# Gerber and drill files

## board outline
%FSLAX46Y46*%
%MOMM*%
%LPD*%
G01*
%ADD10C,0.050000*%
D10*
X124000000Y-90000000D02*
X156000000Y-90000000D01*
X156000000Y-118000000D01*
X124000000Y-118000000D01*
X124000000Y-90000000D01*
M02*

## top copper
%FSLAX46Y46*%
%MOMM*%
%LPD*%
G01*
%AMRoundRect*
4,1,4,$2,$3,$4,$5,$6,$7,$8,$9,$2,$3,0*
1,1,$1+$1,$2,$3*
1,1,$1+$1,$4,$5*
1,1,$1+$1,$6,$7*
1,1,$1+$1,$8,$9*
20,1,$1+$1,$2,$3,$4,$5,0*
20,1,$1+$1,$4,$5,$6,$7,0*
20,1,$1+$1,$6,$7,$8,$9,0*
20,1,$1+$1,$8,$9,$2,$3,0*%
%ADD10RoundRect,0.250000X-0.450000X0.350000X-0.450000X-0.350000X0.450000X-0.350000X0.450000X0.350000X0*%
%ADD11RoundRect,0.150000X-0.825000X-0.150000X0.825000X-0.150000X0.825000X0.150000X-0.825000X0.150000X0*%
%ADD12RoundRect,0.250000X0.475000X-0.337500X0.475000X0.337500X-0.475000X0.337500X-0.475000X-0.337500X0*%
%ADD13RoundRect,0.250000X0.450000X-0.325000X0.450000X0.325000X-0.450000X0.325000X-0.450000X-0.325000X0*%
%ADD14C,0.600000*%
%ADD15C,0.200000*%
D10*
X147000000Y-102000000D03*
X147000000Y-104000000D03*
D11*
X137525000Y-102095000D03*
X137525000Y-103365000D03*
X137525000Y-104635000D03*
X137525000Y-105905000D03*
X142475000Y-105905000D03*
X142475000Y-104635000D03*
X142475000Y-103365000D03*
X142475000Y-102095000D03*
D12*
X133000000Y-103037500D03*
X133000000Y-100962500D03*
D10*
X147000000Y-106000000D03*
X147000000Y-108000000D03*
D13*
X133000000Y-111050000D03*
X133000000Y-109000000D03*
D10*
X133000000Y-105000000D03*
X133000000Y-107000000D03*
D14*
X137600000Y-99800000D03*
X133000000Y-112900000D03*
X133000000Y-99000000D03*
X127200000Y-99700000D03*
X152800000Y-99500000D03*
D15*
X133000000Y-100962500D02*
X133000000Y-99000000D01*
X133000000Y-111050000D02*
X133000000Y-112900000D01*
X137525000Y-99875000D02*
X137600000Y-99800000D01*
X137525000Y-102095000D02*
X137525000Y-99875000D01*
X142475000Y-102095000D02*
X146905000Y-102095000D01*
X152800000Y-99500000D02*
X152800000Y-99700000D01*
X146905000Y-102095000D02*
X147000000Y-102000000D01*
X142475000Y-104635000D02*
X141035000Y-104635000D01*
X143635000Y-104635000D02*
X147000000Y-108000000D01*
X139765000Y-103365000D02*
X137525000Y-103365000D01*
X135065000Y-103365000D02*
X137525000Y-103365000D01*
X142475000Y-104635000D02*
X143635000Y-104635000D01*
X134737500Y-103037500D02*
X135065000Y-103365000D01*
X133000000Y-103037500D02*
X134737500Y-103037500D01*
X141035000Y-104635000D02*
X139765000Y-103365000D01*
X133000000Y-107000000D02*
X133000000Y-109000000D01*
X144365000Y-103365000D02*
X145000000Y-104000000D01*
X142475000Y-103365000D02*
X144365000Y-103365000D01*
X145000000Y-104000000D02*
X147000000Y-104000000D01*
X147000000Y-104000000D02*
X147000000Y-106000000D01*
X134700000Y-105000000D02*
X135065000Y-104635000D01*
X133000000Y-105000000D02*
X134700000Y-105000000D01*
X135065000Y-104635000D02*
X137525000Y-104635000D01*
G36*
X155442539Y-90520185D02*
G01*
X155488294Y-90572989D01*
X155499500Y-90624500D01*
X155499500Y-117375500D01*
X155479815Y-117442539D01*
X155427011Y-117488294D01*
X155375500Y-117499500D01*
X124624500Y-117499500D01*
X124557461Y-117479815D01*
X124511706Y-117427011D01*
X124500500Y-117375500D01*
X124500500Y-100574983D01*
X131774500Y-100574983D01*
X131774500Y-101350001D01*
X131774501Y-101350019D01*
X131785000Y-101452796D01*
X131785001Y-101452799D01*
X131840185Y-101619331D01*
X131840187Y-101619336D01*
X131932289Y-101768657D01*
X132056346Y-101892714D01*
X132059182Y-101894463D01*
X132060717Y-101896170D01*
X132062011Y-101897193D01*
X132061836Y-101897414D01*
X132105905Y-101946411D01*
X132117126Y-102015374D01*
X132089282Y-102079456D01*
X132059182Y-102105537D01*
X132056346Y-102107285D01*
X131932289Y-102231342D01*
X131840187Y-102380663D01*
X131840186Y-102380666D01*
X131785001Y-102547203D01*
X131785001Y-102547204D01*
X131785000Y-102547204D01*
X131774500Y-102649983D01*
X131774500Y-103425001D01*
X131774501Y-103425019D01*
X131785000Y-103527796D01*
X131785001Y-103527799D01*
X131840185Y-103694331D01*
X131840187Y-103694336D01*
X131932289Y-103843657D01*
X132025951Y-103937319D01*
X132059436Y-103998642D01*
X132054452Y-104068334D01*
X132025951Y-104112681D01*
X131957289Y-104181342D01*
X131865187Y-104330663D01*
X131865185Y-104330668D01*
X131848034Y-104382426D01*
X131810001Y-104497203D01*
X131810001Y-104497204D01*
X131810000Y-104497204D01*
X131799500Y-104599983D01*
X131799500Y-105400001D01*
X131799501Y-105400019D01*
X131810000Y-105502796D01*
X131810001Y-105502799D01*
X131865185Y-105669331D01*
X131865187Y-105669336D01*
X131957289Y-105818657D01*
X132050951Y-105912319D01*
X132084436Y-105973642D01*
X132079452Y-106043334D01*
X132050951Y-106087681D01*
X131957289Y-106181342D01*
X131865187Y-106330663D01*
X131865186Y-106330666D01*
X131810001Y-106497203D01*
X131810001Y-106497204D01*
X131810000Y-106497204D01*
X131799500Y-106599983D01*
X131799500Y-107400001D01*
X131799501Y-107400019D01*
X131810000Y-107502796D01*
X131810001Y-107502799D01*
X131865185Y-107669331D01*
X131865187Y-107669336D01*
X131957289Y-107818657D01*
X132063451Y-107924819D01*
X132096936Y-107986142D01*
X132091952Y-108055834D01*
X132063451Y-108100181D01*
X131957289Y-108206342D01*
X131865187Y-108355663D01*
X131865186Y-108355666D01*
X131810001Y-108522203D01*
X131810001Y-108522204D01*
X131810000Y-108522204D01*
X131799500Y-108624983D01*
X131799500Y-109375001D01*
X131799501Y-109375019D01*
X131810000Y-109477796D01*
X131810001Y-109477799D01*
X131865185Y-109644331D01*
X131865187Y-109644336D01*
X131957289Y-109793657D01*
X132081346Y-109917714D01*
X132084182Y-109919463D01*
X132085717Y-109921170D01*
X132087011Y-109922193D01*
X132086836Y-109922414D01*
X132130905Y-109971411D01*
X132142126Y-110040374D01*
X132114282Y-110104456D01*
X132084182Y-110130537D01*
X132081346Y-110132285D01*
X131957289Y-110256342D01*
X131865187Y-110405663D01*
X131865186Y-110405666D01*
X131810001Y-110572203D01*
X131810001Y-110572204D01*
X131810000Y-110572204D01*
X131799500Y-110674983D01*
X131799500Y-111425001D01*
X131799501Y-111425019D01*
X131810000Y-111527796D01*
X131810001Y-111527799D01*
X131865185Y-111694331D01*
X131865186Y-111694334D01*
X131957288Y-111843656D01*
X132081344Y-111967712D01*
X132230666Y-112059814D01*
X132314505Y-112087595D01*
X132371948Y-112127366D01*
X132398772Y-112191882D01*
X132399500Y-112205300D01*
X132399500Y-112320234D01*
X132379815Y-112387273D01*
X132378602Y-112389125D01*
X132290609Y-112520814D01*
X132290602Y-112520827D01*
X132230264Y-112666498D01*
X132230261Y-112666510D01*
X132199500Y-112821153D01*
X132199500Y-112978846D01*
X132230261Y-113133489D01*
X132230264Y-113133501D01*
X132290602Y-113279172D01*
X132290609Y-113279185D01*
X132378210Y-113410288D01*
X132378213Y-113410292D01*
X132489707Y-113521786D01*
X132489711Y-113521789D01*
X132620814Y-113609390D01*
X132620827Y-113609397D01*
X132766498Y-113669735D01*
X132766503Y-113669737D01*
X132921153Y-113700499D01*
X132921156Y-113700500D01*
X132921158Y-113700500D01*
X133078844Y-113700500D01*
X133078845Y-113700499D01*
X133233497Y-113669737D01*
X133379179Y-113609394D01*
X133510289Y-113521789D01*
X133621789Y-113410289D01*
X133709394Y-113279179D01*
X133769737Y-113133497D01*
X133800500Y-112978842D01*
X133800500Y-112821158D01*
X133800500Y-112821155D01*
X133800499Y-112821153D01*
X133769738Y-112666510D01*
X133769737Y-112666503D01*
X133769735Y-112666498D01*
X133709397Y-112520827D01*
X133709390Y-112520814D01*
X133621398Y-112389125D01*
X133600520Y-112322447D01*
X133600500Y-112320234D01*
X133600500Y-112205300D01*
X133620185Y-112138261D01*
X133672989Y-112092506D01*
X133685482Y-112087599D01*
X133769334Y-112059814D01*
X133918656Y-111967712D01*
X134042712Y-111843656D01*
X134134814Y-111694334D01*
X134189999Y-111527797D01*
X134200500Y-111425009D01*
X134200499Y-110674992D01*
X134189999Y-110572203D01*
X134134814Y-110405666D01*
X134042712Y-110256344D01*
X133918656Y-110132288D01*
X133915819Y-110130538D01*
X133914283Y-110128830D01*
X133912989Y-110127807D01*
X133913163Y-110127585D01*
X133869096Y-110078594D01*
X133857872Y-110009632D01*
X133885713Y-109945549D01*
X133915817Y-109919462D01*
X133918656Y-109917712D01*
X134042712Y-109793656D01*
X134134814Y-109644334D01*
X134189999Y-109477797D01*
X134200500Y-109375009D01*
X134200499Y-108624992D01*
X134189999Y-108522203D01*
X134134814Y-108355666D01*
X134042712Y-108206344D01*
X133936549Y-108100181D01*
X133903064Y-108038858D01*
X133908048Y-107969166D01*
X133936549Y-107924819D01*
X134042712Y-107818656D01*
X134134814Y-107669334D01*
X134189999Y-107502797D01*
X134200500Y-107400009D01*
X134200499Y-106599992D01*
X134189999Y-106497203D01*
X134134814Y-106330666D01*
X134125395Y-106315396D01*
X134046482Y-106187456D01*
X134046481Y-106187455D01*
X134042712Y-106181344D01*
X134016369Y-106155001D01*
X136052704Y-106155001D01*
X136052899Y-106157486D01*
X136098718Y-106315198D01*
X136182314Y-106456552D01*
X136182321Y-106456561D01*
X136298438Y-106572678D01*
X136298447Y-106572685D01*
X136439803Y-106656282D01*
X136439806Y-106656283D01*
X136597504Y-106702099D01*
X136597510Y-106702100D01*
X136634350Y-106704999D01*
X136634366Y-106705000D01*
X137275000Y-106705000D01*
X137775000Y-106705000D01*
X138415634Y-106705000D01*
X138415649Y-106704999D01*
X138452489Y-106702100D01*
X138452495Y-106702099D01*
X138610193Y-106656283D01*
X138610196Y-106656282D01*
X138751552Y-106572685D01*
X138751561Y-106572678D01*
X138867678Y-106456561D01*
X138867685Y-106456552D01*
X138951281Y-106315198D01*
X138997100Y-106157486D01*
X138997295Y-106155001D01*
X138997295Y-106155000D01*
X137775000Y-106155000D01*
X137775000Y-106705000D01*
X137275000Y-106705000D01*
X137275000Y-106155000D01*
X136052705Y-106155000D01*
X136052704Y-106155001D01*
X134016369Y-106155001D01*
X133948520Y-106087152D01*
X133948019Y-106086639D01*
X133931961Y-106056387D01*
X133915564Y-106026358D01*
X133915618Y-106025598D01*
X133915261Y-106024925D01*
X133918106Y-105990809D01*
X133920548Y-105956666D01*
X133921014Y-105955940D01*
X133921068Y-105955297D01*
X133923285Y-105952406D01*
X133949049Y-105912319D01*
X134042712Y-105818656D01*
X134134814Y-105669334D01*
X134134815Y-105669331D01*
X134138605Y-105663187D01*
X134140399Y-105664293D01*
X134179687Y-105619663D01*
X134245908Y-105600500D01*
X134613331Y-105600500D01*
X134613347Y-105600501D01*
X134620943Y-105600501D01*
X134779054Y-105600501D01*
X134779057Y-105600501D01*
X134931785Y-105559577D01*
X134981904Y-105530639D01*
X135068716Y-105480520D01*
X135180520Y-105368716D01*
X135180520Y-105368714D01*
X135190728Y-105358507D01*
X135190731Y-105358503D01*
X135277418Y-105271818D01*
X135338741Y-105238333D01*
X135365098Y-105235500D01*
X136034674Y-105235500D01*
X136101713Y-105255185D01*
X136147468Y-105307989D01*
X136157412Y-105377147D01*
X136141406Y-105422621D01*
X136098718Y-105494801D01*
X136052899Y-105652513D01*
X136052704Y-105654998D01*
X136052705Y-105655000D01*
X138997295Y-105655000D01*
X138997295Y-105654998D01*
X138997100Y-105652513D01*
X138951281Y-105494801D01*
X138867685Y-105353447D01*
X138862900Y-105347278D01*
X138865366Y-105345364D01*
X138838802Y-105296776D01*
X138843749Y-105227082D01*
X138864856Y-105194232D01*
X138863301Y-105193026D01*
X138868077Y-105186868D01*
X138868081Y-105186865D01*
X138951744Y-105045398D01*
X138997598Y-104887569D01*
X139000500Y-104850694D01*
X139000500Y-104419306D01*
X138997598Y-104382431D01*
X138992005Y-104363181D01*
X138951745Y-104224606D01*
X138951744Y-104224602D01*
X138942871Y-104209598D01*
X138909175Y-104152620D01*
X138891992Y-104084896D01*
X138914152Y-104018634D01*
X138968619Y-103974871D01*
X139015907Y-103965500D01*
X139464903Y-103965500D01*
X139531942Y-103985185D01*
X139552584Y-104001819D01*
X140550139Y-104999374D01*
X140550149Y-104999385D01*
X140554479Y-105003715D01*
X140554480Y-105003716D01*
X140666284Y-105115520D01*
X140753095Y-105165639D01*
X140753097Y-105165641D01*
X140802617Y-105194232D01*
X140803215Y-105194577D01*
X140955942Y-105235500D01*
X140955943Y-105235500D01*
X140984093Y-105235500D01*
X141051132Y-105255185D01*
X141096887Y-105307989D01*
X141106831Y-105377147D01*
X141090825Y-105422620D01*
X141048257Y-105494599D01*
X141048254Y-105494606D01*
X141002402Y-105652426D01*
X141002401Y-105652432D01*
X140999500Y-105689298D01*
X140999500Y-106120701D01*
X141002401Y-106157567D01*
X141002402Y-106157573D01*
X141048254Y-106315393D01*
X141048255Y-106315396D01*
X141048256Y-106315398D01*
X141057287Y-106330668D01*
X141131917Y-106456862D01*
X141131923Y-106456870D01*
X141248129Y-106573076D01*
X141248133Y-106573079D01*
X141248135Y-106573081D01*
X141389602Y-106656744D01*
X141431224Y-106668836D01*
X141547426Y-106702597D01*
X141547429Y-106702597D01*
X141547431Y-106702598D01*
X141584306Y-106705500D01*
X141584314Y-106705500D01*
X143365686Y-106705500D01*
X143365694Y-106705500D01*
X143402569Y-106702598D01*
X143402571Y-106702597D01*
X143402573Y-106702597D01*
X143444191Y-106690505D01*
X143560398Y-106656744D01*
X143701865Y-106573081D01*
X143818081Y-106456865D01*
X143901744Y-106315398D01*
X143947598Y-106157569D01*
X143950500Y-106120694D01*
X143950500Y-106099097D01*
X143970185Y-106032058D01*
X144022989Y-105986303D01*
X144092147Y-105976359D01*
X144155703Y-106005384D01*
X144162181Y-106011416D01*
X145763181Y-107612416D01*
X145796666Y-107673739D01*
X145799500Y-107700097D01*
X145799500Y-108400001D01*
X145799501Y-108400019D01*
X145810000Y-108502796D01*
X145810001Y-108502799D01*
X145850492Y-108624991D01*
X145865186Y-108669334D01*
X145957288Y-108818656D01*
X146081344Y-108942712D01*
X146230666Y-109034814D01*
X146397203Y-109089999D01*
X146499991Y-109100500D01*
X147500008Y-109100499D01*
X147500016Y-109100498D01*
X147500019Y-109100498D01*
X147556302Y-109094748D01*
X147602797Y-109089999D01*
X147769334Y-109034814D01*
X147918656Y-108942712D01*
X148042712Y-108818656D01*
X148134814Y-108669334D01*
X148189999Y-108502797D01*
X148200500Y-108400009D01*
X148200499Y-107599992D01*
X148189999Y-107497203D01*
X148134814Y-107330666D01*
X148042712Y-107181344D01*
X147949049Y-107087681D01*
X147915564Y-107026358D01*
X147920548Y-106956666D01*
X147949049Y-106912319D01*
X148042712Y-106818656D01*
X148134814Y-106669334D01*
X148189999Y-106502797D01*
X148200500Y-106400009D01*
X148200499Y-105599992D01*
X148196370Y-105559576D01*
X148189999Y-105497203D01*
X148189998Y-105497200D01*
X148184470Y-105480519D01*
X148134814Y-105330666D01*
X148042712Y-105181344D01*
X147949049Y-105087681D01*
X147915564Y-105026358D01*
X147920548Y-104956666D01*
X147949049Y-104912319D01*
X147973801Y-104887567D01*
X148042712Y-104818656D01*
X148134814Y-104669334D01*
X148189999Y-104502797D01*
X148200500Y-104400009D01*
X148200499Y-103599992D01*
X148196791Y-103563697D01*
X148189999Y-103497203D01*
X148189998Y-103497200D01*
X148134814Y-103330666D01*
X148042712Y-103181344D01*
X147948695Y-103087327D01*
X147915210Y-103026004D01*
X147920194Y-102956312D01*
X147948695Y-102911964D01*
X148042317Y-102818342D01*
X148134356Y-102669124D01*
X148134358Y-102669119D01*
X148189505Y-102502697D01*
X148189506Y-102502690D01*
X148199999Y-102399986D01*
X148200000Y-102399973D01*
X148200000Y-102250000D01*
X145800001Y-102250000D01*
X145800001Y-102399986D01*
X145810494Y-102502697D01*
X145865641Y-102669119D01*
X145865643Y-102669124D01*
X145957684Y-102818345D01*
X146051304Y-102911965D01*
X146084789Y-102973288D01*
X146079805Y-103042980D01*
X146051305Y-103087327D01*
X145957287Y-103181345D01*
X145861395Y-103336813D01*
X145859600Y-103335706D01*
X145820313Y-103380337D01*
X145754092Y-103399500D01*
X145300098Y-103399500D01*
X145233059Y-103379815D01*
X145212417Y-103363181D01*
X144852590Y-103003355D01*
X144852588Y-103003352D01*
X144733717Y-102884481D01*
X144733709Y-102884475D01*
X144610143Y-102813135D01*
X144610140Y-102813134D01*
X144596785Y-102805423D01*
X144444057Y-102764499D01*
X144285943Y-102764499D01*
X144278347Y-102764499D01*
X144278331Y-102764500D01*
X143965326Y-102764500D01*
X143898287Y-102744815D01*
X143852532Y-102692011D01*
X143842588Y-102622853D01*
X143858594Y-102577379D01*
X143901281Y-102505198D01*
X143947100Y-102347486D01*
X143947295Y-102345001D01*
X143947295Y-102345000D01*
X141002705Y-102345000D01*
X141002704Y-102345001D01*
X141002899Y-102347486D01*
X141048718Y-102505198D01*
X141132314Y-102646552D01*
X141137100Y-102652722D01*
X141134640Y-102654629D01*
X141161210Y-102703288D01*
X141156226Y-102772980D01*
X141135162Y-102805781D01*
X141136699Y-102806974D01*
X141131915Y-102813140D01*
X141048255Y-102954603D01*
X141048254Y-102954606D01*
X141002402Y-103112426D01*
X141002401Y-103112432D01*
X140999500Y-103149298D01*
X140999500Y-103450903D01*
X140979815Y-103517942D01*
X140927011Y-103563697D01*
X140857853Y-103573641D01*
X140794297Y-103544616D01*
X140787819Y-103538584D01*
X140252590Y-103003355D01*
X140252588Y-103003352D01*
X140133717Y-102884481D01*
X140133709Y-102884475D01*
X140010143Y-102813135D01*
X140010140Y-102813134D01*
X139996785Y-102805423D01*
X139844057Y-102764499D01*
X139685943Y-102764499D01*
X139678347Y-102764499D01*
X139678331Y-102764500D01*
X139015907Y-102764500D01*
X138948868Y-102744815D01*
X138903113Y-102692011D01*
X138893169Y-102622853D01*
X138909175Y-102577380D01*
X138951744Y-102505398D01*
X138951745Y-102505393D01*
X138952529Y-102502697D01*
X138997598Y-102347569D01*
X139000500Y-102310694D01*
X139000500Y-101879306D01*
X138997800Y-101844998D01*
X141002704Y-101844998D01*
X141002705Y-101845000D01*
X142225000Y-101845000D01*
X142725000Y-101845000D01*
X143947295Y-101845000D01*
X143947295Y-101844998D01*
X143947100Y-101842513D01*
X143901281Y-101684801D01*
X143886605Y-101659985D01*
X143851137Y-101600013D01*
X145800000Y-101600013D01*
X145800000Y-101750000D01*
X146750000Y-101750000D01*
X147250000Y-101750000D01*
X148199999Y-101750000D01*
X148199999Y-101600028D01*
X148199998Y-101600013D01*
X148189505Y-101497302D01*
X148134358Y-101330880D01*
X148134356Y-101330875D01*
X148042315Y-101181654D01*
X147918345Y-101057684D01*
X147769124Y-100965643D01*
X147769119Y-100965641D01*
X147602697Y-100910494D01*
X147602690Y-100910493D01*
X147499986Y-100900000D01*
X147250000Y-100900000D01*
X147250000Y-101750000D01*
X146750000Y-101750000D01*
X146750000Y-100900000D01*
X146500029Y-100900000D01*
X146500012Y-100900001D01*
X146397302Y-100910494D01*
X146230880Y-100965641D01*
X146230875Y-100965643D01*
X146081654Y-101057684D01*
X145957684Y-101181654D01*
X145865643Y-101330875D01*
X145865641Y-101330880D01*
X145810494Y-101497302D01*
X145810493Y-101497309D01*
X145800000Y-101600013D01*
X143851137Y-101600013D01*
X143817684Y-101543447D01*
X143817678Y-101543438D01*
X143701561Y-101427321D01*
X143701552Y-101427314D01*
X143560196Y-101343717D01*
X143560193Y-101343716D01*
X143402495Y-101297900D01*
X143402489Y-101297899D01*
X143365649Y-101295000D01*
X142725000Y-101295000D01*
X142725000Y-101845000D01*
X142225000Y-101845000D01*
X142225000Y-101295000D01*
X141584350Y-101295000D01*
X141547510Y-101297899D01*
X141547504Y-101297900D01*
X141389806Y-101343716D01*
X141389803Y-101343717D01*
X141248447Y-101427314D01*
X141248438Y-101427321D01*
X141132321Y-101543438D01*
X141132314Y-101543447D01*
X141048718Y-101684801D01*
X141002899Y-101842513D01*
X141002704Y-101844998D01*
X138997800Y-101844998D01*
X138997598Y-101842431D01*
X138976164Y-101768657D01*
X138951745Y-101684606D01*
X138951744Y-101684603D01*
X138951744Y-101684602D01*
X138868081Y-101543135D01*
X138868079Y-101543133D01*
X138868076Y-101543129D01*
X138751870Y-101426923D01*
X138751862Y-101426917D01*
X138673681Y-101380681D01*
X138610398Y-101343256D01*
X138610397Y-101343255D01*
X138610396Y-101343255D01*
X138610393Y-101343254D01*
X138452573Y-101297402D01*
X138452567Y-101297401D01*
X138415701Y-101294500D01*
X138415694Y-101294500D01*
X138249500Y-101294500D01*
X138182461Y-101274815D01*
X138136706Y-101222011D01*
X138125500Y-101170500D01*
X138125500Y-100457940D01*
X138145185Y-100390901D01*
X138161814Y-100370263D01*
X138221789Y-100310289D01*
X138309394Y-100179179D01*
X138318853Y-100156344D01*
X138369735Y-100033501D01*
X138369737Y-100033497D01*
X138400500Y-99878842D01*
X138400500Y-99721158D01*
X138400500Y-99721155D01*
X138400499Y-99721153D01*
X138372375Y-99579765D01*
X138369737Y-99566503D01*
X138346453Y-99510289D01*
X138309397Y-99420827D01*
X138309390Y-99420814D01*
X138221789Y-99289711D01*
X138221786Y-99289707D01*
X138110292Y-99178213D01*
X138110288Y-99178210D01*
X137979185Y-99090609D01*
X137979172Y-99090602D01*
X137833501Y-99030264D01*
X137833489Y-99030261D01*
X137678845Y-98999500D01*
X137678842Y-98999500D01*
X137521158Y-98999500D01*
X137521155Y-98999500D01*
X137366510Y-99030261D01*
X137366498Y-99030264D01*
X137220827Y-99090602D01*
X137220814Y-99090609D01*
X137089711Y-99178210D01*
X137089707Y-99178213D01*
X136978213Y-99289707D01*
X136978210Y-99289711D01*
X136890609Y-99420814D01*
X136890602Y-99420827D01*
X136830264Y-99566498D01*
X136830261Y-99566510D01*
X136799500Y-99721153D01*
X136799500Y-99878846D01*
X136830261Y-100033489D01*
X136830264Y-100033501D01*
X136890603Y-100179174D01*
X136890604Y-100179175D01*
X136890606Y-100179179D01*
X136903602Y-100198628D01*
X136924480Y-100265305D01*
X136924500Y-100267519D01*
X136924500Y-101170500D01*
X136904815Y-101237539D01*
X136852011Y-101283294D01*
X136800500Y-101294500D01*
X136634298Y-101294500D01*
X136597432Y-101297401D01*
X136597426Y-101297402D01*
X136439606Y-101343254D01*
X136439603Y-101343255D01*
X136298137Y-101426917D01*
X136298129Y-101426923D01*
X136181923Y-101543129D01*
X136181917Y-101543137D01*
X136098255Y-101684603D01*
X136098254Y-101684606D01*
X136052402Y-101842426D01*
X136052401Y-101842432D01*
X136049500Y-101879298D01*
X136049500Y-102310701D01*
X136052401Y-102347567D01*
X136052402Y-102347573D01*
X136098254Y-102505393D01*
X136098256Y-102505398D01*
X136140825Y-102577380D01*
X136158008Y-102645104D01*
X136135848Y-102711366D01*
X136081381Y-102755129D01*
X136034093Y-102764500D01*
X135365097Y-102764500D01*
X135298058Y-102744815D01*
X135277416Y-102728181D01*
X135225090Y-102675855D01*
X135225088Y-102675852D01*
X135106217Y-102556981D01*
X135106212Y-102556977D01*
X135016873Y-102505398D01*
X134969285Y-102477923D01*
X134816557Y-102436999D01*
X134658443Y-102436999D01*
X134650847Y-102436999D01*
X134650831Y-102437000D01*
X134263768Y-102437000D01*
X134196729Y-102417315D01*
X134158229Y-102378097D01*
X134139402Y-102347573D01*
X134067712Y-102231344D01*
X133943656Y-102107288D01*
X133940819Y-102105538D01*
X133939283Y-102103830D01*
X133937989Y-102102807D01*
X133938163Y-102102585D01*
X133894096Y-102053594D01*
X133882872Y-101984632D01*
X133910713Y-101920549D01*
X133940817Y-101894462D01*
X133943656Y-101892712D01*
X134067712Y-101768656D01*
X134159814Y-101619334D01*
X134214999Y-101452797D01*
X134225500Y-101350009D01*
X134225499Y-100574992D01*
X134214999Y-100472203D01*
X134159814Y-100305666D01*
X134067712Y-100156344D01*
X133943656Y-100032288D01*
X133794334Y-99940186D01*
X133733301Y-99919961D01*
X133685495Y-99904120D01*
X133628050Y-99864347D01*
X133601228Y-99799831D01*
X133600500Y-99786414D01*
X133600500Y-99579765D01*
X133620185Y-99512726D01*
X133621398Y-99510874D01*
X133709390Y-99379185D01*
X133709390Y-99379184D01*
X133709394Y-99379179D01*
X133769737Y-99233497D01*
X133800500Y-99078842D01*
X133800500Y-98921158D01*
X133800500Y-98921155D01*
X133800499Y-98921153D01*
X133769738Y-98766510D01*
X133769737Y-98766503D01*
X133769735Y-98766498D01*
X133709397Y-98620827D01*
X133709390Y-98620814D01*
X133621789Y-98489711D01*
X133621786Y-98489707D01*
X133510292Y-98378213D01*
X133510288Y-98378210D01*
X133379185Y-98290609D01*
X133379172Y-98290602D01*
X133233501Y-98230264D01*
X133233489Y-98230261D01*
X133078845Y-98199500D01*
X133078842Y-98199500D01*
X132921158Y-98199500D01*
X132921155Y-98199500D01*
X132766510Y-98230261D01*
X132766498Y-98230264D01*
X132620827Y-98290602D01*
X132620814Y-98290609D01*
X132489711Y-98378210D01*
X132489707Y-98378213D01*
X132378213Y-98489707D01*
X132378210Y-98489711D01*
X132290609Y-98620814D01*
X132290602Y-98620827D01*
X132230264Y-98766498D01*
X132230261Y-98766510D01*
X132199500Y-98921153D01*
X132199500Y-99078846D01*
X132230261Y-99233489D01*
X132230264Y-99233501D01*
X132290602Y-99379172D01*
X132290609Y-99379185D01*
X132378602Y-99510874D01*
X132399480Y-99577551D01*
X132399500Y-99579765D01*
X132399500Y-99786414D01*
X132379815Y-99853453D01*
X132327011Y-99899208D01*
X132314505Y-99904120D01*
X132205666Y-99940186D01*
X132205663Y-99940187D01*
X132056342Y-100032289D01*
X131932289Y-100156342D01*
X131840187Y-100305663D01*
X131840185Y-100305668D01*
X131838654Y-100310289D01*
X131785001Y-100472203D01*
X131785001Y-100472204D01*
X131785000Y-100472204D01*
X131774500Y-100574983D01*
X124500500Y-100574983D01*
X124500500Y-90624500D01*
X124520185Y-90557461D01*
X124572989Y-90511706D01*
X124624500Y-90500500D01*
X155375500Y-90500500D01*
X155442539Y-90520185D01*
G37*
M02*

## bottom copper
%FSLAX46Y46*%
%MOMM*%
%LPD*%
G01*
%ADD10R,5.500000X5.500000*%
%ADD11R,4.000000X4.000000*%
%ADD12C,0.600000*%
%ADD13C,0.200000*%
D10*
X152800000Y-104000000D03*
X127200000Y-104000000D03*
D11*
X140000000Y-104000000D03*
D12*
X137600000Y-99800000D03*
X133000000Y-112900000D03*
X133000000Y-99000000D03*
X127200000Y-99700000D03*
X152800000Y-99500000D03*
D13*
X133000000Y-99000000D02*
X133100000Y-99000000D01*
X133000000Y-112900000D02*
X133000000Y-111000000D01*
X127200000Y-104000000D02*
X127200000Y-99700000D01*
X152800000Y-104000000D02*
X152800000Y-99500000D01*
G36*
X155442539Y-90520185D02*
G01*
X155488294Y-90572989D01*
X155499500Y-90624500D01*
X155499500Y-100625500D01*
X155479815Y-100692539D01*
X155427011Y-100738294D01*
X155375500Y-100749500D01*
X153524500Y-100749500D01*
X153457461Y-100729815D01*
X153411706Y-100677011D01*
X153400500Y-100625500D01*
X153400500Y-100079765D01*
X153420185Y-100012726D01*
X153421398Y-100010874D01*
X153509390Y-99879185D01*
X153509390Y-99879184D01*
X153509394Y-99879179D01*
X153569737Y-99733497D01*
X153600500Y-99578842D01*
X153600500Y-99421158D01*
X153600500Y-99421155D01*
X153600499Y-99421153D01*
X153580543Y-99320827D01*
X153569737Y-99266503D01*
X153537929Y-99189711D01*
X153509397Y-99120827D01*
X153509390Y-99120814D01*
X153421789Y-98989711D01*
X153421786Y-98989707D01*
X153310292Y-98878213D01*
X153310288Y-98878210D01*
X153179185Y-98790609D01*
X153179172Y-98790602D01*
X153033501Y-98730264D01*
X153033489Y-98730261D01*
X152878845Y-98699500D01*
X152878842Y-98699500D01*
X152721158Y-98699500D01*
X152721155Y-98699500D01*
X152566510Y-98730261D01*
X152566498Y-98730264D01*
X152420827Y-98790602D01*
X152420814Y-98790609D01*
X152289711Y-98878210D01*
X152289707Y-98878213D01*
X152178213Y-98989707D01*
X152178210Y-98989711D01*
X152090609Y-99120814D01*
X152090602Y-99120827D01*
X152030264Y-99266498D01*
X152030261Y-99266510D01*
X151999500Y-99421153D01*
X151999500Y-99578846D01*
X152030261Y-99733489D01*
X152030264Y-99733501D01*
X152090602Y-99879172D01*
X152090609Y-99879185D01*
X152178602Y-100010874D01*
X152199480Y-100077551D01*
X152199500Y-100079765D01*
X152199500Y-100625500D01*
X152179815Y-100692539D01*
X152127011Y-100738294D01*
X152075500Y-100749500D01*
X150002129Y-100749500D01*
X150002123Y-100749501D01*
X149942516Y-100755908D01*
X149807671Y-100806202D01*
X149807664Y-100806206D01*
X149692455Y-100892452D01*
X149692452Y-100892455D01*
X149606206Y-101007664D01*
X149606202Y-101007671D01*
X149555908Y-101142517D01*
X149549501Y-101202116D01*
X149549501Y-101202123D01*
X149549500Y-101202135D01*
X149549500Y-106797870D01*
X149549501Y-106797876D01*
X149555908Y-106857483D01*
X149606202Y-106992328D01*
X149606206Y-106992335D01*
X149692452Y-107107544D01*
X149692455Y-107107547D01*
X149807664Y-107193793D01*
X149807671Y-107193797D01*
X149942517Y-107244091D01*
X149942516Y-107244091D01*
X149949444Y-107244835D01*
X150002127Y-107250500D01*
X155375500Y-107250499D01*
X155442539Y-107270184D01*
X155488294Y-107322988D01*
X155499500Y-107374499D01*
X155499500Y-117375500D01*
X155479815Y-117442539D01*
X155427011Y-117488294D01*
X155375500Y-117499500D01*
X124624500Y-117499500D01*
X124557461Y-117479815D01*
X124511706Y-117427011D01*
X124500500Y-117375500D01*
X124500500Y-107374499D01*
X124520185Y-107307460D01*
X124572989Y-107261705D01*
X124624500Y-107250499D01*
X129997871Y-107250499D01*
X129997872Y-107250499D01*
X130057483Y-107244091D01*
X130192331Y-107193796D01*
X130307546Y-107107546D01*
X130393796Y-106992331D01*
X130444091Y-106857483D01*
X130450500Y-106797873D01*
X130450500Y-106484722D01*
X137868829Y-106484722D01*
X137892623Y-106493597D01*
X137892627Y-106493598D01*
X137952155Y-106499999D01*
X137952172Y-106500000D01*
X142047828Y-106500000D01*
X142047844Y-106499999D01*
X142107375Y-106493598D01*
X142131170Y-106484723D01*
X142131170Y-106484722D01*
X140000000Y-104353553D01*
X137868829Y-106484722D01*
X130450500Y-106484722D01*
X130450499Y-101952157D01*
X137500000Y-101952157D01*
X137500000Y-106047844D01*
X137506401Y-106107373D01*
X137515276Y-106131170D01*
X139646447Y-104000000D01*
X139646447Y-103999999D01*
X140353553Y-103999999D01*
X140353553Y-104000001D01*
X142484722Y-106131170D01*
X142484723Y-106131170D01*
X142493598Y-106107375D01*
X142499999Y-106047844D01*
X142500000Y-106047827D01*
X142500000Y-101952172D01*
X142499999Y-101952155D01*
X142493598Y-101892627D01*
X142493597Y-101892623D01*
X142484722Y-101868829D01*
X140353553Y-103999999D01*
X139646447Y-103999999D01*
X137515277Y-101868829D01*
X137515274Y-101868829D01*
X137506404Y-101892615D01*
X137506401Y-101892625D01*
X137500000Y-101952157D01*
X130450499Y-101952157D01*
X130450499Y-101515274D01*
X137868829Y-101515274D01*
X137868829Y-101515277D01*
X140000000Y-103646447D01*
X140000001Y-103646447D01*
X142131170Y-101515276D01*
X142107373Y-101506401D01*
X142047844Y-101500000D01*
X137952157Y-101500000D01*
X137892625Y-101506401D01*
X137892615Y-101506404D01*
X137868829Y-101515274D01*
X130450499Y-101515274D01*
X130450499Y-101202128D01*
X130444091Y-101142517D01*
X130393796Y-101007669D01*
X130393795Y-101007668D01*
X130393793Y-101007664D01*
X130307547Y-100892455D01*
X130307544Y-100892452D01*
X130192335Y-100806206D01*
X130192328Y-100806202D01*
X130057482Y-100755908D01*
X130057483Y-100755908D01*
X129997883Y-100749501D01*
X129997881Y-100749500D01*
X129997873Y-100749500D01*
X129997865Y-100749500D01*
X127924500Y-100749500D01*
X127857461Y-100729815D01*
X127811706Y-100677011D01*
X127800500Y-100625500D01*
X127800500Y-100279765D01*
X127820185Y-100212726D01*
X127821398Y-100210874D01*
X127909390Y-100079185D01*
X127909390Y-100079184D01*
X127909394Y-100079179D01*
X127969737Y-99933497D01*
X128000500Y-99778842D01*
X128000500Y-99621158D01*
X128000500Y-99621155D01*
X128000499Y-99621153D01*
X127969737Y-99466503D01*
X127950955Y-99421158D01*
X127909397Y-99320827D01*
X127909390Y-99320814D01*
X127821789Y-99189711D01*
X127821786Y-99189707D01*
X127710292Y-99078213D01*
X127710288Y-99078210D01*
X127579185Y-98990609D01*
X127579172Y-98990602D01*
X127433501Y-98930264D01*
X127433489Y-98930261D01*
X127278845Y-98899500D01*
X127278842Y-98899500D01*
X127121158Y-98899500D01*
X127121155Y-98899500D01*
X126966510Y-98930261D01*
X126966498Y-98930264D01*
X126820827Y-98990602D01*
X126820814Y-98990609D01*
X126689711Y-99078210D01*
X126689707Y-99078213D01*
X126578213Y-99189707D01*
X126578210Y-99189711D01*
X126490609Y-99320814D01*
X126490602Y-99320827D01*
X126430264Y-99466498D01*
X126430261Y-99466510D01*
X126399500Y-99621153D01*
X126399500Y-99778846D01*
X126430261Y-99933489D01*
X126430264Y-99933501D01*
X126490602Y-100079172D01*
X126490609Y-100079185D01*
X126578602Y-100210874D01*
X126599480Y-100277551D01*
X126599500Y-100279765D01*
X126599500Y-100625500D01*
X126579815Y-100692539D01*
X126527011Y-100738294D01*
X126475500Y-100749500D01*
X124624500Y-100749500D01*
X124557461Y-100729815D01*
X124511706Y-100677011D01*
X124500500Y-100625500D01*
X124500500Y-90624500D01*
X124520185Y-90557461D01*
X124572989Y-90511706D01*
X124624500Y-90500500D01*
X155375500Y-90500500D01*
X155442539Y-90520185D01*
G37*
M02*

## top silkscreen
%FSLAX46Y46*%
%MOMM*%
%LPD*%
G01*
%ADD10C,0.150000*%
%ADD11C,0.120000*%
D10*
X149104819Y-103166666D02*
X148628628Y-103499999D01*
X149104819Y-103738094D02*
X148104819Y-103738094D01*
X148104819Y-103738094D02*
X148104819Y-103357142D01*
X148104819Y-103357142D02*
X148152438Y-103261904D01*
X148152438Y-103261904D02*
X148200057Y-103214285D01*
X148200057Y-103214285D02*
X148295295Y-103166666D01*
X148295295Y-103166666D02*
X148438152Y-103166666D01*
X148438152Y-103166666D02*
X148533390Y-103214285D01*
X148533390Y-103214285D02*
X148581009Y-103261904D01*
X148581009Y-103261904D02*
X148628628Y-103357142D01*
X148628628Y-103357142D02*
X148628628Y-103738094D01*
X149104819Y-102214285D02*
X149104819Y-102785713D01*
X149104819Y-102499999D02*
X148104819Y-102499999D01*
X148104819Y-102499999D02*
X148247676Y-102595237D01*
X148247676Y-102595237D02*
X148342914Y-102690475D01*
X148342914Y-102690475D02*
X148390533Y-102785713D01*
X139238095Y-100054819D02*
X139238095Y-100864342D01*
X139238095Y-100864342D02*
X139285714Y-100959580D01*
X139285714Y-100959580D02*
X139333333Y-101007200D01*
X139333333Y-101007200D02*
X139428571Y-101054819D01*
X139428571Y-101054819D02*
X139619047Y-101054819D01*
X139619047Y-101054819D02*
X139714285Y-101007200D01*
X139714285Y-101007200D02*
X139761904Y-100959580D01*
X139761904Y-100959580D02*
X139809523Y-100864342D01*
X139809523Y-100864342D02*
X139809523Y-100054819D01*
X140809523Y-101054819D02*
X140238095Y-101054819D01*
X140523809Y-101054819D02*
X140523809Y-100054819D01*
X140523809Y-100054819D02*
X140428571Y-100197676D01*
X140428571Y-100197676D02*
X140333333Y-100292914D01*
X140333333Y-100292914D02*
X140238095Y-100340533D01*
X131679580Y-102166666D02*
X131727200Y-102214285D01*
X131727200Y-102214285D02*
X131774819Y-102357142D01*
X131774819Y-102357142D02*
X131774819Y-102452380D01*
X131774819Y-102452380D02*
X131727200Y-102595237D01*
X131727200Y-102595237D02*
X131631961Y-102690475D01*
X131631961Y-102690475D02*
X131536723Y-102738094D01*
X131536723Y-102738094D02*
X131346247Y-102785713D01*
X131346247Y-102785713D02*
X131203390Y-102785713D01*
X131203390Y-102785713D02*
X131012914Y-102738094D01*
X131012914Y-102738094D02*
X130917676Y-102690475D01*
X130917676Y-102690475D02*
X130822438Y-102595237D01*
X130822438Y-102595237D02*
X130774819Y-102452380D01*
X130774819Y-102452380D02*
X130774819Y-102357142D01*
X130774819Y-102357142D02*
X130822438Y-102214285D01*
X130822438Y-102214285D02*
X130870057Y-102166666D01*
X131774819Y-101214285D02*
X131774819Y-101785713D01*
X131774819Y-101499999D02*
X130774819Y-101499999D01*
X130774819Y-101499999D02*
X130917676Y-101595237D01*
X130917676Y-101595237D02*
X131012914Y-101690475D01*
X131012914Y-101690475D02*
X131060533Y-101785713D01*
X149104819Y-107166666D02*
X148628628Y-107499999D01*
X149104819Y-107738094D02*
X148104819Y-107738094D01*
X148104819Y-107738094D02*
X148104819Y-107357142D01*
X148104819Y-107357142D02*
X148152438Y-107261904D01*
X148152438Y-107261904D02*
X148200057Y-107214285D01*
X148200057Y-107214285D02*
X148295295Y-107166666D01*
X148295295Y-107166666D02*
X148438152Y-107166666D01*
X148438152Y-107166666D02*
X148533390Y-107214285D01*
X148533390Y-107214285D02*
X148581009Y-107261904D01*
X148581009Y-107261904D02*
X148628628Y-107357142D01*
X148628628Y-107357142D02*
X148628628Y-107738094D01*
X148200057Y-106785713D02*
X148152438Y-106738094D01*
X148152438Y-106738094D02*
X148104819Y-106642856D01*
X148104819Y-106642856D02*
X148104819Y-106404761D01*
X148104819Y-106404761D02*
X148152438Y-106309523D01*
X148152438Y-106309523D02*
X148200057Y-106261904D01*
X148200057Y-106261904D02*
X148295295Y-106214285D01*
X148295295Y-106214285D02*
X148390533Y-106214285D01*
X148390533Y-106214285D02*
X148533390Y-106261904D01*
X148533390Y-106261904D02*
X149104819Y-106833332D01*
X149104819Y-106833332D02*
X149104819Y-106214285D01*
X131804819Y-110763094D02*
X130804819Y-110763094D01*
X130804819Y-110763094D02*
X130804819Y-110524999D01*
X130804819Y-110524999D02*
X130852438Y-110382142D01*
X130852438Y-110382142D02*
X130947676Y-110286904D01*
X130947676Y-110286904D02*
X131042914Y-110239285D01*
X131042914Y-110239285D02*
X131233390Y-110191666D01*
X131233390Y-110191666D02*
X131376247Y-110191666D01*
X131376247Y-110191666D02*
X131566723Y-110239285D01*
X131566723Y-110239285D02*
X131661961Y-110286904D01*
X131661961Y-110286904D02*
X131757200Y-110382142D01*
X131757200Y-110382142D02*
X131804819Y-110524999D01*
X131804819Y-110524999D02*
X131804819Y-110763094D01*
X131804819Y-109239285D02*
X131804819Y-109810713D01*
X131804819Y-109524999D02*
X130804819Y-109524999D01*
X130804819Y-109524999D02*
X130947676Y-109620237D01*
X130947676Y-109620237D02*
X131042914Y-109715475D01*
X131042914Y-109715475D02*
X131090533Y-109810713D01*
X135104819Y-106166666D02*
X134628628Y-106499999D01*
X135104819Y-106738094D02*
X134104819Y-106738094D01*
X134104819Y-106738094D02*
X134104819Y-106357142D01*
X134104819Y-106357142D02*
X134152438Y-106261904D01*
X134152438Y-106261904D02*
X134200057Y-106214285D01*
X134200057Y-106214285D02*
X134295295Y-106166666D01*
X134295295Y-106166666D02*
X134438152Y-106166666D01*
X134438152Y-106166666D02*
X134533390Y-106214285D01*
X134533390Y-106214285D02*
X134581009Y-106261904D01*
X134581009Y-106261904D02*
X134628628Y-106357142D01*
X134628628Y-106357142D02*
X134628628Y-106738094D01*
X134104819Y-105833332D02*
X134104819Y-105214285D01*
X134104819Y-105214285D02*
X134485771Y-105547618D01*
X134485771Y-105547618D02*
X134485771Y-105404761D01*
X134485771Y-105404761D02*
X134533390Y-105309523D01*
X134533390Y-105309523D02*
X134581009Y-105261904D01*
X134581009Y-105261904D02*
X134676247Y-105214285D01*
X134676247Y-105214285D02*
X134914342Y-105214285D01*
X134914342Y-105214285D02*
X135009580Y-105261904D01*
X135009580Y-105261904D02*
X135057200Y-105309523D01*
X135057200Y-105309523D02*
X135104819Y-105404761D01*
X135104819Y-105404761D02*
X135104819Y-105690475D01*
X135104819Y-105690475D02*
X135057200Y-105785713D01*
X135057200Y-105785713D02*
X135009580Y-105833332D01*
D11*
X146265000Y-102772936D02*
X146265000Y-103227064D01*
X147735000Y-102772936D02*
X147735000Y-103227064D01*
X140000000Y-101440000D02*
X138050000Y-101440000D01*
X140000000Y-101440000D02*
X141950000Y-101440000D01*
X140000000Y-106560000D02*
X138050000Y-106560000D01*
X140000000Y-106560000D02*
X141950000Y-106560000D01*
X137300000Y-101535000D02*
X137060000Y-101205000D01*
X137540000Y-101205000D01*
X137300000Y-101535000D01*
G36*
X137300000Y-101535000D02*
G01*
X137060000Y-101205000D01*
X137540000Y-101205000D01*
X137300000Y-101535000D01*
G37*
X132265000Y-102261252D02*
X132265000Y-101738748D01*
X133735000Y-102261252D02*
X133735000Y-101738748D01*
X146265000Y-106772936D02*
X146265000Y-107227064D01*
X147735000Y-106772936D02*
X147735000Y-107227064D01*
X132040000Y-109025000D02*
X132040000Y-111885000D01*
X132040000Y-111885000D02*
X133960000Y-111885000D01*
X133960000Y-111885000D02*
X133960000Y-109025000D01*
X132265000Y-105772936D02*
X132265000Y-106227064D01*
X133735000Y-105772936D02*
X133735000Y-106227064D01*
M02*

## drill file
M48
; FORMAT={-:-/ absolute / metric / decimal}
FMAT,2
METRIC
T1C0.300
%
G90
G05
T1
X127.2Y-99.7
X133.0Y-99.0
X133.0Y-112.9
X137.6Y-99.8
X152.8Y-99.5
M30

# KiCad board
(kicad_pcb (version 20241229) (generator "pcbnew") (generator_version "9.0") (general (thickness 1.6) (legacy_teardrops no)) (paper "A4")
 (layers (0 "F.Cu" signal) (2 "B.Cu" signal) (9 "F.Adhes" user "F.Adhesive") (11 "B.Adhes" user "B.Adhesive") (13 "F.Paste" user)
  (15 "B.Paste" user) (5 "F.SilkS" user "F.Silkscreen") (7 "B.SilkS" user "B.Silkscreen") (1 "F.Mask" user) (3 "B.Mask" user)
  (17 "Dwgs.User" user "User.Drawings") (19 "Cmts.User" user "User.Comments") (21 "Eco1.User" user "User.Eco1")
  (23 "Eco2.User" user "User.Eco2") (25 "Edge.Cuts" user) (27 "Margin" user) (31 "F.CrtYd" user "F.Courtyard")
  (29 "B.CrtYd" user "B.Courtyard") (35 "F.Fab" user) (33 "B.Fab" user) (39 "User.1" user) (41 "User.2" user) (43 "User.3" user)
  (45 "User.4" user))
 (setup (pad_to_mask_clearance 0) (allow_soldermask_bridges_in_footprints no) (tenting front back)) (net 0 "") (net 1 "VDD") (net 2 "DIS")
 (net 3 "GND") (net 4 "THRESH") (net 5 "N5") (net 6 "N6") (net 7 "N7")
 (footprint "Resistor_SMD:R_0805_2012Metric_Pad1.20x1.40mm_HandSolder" (layer "F.Cu") (at 147 103 -90)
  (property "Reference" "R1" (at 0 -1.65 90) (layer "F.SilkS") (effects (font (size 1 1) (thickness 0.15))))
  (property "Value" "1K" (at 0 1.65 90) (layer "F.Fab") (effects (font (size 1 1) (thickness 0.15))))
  (fp_line (start -0.227064 0.735) (end 0.227064 0.735) (stroke (width 0.12) (type solid)) (layer "F.SilkS"))
  (fp_line (start -0.227064 -0.735) (end 0.227064 -0.735) (stroke (width 0.12) (type solid)) (layer "F.SilkS"))
  (pad "1" smd roundrect (at -1 0 270) (size 1.2 1.4) (layers "F.Cu" "F.Mask" "F.Paste") (roundrect_rratio 0.208333) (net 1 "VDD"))
  (pad "2" smd roundrect (at 1 0 270) (size 1.2 1.4) (layers "F.Cu" "F.Mask" "F.Paste") (roundrect_rratio 0.208333) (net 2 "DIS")))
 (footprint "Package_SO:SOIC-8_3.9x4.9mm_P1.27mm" (layer "F.Cu") (at 140 104)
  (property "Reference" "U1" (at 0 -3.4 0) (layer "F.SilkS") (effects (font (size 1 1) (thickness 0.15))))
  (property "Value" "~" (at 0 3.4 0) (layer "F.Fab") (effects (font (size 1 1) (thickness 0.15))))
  (fp_line (start 0 -2.56) (end -1.95 -2.56) (stroke (width 0.12) (type solid)) (layer "F.SilkS"))
  (fp_line (start 0 -2.56) (end 1.95 -2.56) (stroke (width 0.12) (type solid)) (layer "F.SilkS"))
  (fp_line (start 0 2.56) (end -1.95 2.56) (stroke (width 0.12) (type solid)) (layer "F.SilkS"))
  (fp_line (start 0 2.56) (end 1.95 2.56) (stroke (width 0.12) (type solid)) (layer "F.SilkS"))
  (fp_poly (pts (xy -2.7 -2.465) (xy -2.94 -2.795) (xy -2.46 -2.795)) (stroke (width 0.12) (type solid)) (fill yes) (layer "F.SilkS"))
  (pad "1" smd roundrect (at -2.475 -1.905) (size 1.95 0.6) (layers "F.Cu" "F.Mask" "F.Paste") (roundrect_rratio 0.25) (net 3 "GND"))
  (pad "2" smd roundrect (at -2.475 -0.635) (size 1.95 0.6) (layers "F.Cu" "F.Mask" "F.Paste") (roundrect_rratio 0.25) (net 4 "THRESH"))
  (pad "3" smd roundrect (at -2.475 0.635) (size 1.95 0.6) (layers "F.Cu" "F.Mask" "F.Paste") (roundrect_rratio 0.25) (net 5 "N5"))
  (pad "4" smd roundrect (at -2.475 1.905) (size 1.95 0.6) (layers "F.Cu" "F.Mask" "F.Paste") (roundrect_rratio 0.25) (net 1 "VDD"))
  (pad "5" smd roundrect (at 2.475 1.905) (size 1.95 0.6) (layers "F.Cu" "F.Mask" "F.Paste") (roundrect_rratio 0.25) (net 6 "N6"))
  (pad "6" smd roundrect (at 2.475 0.635) (size 1.95 0.6) (layers "F.Cu" "F.Mask" "F.Paste") (roundrect_rratio 0.25) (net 4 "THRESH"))
  (pad "7" smd roundrect (at 2.475 -0.635) (size 1.95 0.6) (layers "F.Cu" "F.Mask" "F.Paste") (roundrect_rratio 0.25) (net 2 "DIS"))
  (pad "8" smd roundrect (at 2.475 -1.905) (size 1.95 0.6) (layers "F.Cu" "F.Mask" "F.Paste") (roundrect_rratio 0.25) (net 1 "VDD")))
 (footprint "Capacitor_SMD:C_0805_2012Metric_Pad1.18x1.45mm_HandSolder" (layer "F.Cu") (at 133 102 90)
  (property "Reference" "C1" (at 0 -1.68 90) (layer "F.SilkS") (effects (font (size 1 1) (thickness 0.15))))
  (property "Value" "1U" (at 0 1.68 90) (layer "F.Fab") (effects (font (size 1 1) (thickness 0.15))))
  (fp_line (start -0.261252 -0.735) (end 0.261252 -0.735) (stroke (width 0.12) (type solid)) (layer "F.SilkS"))
  (fp_line (start -0.261252 0.735) (end 0.261252 0.735) (stroke (width 0.12) (type solid)) (layer "F.SilkS"))
  (pad "1" smd roundrect (at -1.0375 0 90) (size 1.175 1.45) (layers "F.Cu" "F.Mask" "F.Paste") (roundrect_rratio 0.212766) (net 4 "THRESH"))
  (pad "2" smd roundrect (at 1.0375 0 90) (size 1.175 1.45) (layers "F.Cu" "F.Mask" "F.Paste") (roundrect_rratio 0.212766) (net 3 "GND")))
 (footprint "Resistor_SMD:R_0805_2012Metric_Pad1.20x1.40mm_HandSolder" (layer "F.Cu") (at 147 107 -90)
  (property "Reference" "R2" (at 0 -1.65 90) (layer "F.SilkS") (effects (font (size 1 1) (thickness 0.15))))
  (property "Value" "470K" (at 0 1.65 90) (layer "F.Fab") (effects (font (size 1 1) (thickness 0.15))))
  (fp_line (start -0.227064 0.735) (end 0.227064 0.735) (stroke (width 0.12) (type solid)) (layer "F.SilkS"))
  (fp_line (start -0.227064 -0.735) (end 0.227064 -0.735) (stroke (width 0.12) (type solid)) (layer "F.SilkS"))
  (pad "1" smd roundrect (at -1 0 270) (size 1.2 1.4) (layers "F.Cu" "F.Mask" "F.Paste") (roundrect_rratio 0.208333) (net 2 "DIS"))
  (pad "2" smd roundrect (at 1 0 270) (size 1.2 1.4) (layers "F.Cu" "F.Mask" "F.Paste") (roundrect_rratio 0.208333) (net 4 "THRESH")))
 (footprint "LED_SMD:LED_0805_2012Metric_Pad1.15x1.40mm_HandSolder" (layer "F.Cu") (at 133 110.025 90)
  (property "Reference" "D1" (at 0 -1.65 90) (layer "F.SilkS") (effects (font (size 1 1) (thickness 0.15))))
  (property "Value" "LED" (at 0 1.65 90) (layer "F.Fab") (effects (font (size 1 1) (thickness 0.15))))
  (fp_line (start 1 -0.96) (end -1.86 -0.96) (stroke (width 0.12) (type solid)) (layer "F.SilkS"))
  (fp_line (start -1.86 -0.96) (end -1.86 0.96) (stroke (width 0.12) (type solid)) (layer "F.SilkS"))
  (fp_line (start -1.86 0.96) (end 1 0.96) (stroke (width 0.12) (type solid)) (layer "F.SilkS"))
  (pad "1" smd roundrect (at -1.025 0 90) (size 1.15 1.4) (layers "F.Cu" "F.Mask" "F.Paste") (roundrect_rratio 0.217391) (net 3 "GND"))
  (pad "2" smd roundrect (at 1.025 0 90) (size 1.15 1.4) (layers "F.Cu" "F.Mask" "F.Paste") (roundrect_rratio 0.217391) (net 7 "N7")))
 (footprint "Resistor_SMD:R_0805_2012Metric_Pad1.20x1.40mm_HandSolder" (layer "F.Cu") (at 133 106 -90)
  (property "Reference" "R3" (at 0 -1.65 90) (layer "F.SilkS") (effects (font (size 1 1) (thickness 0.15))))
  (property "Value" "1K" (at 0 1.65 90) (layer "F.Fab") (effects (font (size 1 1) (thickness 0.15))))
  (fp_line (start -0.227064 0.735) (end 0.227064 0.735) (stroke (width 0.12) (type solid)) (layer "F.SilkS"))
  (fp_line (start -0.227064 -0.735) (end 0.227064 -0.735) (stroke (width 0.12) (type solid)) (layer "F.SilkS"))
  (pad "1" smd roundrect (at -1 0 270) (size 1.2 1.4) (layers "F.Cu" "F.Mask" "F.Paste") (roundrect_rratio 0.208333) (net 5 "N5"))
  (pad "2" smd roundrect (at 1 0 270) (size 1.2 1.4) (layers "F.Cu" "F.Mask" "F.Paste") (roundrect_rratio 0.208333) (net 7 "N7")))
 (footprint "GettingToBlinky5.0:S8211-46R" (layer "B.Cu") (at 140 104 180)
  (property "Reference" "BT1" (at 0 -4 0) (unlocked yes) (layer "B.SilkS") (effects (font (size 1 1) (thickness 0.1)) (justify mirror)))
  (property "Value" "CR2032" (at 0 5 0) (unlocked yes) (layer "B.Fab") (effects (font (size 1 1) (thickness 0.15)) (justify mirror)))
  (pad "1" smd rect (at -12.8 0 180) (size 5.5 5.5) (layers "B.Cu" "B.Mask" "B.Paste") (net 1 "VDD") (thermal_bridge_angle 45))
  (pad "2" smd rect (at 12.8 0 180) (size 5.5 5.5) (layers "B.Cu" "B.Mask" "B.Paste") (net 1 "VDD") (thermal_bridge_angle 45))
  (pad "3" smd rect (at 0 0 180) (size 4 4) (layers "B.Cu" "B.Mask" "B.Paste") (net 3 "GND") (thermal_bridge_angle 45)))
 (gr_rect (start 124 90) (end 156 118) (stroke (width 0.05) (type default)) (fill no) (layer "Edge.Cuts"))
 (segment (start 133 100.9625) (end 133 99) (width 0.2) (layer "F.Cu") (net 3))
 (segment (start 133 111.05) (end 133 112.9) (width 0.2) (layer "F.Cu") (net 3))
 (segment (start 137.525 99.875) (end 137.6 99.8) (width 0.2) (layer "F.Cu") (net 3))
 (segment (start 137.525 102.095) (end 137.525 99.875) (width 0.2) (layer "F.Cu") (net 3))
 (via (at 137.6 99.8) (size 0.6) (drill 0.3) (layers "F.Cu" "B.Cu") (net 3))
 (via (at 133 112.9) (size 0.6) (drill 0.3) (layers "F.Cu" "B.Cu") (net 3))
 (via (at 133 99) (size 0.6) (drill 0.3) (layers "F.Cu" "B.Cu") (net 3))
 (segment (start 133 99) (end 133.1 99) (width 0.2) (layer "B.Cu") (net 3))
 (segment (start 133 112.9) (end 133 111) (width 0.2) (layer "B.Cu") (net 3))
 (segment (start 142.475 102.095) (end 146.905 102.095) (width 0.2) (layer "F.Cu") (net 1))
 (segment (start 152.8 99.5) (end 152.8 99.7) (width 0.2) (layer "F.Cu") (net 1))
 (segment (start 146.905 102.095) (end 147 102) (width 0.2) (layer "F.Cu") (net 1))
 (via (at 127.2 99.7) (size 0.6) (drill 0.3) (layers "F.Cu" "B.Cu") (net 1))
 (via (at 152.8 99.5) (size 0.6) (drill 0.3) (layers "F.Cu" "B.Cu") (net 1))
 (segment (start 127.2 104) (end 127.2 99.7) (width 0.2) (layer "B.Cu") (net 1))
 (segment (start 152.8 104) (end 152.8 99.5) (width 0.2) (layer "B.Cu") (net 1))
 (segment (start 142.475 104.635) (end 141.035 104.635) (width 0.2) (layer "F.Cu") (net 4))
 (segment (start 143.635 104.635) (end 147 108) (width 0.2) (layer "F.Cu") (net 4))
 (segment (start 139.765 103.365) (end 137.525 103.365) (width 0.2) (layer "F.Cu") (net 4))
 (segment (start 135.065 103.365) (end 137.525 103.365) (width 0.2) (layer "F.Cu") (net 4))
 (segment (start 142.475 104.635) (end 143.635 104.635) (width 0.2) (layer "F.Cu") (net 4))
 (segment (start 134.7375 103.0375) (end 135.065 103.365) (width 0.2) (layer "F.Cu") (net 4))
 (segment (start 133 103.0375) (end 134.7375 103.0375) (width 0.2) (layer "F.Cu") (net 4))
 (segment (start 141.035 104.635) (end 139.765 103.365) (width 0.2) (layer "F.Cu") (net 4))
 (segment (start 133 107) (end 133 109) (width 0.2) (layer "F.Cu") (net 7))
 (segment (start 144.365 103.365) (end 145 104) (width 0.2) (layer "F.Cu") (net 2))
 (segment (start 142.475 103.365) (end 144.365 103.365) (width 0.2) (layer "F.Cu") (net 2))
 (segment (start 145 104) (end 147 104) (width 0.2) (layer "F.Cu") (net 2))
 (segment (start 147 104) (end 147 106) (width 0.2) (layer "F.Cu") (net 2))
 (segment (start 134.7 105) (end 135.065 104.635) (width 0.2) (layer "F.Cu") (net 5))
 (segment (start 133 105) (end 134.7 105) (width 0.2) (layer "F.Cu") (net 5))
 (segment (start 135.065 104.635) (end 137.525 104.635) (width 0.2) (layer "F.Cu") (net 5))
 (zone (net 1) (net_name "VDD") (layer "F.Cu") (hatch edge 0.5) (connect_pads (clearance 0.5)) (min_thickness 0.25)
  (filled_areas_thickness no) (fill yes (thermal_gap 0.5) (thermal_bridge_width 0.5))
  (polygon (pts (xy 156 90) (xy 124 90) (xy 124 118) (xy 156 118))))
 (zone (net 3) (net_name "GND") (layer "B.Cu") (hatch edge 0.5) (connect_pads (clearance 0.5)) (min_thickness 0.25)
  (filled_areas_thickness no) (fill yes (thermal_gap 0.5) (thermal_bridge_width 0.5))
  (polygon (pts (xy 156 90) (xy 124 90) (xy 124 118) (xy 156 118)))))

